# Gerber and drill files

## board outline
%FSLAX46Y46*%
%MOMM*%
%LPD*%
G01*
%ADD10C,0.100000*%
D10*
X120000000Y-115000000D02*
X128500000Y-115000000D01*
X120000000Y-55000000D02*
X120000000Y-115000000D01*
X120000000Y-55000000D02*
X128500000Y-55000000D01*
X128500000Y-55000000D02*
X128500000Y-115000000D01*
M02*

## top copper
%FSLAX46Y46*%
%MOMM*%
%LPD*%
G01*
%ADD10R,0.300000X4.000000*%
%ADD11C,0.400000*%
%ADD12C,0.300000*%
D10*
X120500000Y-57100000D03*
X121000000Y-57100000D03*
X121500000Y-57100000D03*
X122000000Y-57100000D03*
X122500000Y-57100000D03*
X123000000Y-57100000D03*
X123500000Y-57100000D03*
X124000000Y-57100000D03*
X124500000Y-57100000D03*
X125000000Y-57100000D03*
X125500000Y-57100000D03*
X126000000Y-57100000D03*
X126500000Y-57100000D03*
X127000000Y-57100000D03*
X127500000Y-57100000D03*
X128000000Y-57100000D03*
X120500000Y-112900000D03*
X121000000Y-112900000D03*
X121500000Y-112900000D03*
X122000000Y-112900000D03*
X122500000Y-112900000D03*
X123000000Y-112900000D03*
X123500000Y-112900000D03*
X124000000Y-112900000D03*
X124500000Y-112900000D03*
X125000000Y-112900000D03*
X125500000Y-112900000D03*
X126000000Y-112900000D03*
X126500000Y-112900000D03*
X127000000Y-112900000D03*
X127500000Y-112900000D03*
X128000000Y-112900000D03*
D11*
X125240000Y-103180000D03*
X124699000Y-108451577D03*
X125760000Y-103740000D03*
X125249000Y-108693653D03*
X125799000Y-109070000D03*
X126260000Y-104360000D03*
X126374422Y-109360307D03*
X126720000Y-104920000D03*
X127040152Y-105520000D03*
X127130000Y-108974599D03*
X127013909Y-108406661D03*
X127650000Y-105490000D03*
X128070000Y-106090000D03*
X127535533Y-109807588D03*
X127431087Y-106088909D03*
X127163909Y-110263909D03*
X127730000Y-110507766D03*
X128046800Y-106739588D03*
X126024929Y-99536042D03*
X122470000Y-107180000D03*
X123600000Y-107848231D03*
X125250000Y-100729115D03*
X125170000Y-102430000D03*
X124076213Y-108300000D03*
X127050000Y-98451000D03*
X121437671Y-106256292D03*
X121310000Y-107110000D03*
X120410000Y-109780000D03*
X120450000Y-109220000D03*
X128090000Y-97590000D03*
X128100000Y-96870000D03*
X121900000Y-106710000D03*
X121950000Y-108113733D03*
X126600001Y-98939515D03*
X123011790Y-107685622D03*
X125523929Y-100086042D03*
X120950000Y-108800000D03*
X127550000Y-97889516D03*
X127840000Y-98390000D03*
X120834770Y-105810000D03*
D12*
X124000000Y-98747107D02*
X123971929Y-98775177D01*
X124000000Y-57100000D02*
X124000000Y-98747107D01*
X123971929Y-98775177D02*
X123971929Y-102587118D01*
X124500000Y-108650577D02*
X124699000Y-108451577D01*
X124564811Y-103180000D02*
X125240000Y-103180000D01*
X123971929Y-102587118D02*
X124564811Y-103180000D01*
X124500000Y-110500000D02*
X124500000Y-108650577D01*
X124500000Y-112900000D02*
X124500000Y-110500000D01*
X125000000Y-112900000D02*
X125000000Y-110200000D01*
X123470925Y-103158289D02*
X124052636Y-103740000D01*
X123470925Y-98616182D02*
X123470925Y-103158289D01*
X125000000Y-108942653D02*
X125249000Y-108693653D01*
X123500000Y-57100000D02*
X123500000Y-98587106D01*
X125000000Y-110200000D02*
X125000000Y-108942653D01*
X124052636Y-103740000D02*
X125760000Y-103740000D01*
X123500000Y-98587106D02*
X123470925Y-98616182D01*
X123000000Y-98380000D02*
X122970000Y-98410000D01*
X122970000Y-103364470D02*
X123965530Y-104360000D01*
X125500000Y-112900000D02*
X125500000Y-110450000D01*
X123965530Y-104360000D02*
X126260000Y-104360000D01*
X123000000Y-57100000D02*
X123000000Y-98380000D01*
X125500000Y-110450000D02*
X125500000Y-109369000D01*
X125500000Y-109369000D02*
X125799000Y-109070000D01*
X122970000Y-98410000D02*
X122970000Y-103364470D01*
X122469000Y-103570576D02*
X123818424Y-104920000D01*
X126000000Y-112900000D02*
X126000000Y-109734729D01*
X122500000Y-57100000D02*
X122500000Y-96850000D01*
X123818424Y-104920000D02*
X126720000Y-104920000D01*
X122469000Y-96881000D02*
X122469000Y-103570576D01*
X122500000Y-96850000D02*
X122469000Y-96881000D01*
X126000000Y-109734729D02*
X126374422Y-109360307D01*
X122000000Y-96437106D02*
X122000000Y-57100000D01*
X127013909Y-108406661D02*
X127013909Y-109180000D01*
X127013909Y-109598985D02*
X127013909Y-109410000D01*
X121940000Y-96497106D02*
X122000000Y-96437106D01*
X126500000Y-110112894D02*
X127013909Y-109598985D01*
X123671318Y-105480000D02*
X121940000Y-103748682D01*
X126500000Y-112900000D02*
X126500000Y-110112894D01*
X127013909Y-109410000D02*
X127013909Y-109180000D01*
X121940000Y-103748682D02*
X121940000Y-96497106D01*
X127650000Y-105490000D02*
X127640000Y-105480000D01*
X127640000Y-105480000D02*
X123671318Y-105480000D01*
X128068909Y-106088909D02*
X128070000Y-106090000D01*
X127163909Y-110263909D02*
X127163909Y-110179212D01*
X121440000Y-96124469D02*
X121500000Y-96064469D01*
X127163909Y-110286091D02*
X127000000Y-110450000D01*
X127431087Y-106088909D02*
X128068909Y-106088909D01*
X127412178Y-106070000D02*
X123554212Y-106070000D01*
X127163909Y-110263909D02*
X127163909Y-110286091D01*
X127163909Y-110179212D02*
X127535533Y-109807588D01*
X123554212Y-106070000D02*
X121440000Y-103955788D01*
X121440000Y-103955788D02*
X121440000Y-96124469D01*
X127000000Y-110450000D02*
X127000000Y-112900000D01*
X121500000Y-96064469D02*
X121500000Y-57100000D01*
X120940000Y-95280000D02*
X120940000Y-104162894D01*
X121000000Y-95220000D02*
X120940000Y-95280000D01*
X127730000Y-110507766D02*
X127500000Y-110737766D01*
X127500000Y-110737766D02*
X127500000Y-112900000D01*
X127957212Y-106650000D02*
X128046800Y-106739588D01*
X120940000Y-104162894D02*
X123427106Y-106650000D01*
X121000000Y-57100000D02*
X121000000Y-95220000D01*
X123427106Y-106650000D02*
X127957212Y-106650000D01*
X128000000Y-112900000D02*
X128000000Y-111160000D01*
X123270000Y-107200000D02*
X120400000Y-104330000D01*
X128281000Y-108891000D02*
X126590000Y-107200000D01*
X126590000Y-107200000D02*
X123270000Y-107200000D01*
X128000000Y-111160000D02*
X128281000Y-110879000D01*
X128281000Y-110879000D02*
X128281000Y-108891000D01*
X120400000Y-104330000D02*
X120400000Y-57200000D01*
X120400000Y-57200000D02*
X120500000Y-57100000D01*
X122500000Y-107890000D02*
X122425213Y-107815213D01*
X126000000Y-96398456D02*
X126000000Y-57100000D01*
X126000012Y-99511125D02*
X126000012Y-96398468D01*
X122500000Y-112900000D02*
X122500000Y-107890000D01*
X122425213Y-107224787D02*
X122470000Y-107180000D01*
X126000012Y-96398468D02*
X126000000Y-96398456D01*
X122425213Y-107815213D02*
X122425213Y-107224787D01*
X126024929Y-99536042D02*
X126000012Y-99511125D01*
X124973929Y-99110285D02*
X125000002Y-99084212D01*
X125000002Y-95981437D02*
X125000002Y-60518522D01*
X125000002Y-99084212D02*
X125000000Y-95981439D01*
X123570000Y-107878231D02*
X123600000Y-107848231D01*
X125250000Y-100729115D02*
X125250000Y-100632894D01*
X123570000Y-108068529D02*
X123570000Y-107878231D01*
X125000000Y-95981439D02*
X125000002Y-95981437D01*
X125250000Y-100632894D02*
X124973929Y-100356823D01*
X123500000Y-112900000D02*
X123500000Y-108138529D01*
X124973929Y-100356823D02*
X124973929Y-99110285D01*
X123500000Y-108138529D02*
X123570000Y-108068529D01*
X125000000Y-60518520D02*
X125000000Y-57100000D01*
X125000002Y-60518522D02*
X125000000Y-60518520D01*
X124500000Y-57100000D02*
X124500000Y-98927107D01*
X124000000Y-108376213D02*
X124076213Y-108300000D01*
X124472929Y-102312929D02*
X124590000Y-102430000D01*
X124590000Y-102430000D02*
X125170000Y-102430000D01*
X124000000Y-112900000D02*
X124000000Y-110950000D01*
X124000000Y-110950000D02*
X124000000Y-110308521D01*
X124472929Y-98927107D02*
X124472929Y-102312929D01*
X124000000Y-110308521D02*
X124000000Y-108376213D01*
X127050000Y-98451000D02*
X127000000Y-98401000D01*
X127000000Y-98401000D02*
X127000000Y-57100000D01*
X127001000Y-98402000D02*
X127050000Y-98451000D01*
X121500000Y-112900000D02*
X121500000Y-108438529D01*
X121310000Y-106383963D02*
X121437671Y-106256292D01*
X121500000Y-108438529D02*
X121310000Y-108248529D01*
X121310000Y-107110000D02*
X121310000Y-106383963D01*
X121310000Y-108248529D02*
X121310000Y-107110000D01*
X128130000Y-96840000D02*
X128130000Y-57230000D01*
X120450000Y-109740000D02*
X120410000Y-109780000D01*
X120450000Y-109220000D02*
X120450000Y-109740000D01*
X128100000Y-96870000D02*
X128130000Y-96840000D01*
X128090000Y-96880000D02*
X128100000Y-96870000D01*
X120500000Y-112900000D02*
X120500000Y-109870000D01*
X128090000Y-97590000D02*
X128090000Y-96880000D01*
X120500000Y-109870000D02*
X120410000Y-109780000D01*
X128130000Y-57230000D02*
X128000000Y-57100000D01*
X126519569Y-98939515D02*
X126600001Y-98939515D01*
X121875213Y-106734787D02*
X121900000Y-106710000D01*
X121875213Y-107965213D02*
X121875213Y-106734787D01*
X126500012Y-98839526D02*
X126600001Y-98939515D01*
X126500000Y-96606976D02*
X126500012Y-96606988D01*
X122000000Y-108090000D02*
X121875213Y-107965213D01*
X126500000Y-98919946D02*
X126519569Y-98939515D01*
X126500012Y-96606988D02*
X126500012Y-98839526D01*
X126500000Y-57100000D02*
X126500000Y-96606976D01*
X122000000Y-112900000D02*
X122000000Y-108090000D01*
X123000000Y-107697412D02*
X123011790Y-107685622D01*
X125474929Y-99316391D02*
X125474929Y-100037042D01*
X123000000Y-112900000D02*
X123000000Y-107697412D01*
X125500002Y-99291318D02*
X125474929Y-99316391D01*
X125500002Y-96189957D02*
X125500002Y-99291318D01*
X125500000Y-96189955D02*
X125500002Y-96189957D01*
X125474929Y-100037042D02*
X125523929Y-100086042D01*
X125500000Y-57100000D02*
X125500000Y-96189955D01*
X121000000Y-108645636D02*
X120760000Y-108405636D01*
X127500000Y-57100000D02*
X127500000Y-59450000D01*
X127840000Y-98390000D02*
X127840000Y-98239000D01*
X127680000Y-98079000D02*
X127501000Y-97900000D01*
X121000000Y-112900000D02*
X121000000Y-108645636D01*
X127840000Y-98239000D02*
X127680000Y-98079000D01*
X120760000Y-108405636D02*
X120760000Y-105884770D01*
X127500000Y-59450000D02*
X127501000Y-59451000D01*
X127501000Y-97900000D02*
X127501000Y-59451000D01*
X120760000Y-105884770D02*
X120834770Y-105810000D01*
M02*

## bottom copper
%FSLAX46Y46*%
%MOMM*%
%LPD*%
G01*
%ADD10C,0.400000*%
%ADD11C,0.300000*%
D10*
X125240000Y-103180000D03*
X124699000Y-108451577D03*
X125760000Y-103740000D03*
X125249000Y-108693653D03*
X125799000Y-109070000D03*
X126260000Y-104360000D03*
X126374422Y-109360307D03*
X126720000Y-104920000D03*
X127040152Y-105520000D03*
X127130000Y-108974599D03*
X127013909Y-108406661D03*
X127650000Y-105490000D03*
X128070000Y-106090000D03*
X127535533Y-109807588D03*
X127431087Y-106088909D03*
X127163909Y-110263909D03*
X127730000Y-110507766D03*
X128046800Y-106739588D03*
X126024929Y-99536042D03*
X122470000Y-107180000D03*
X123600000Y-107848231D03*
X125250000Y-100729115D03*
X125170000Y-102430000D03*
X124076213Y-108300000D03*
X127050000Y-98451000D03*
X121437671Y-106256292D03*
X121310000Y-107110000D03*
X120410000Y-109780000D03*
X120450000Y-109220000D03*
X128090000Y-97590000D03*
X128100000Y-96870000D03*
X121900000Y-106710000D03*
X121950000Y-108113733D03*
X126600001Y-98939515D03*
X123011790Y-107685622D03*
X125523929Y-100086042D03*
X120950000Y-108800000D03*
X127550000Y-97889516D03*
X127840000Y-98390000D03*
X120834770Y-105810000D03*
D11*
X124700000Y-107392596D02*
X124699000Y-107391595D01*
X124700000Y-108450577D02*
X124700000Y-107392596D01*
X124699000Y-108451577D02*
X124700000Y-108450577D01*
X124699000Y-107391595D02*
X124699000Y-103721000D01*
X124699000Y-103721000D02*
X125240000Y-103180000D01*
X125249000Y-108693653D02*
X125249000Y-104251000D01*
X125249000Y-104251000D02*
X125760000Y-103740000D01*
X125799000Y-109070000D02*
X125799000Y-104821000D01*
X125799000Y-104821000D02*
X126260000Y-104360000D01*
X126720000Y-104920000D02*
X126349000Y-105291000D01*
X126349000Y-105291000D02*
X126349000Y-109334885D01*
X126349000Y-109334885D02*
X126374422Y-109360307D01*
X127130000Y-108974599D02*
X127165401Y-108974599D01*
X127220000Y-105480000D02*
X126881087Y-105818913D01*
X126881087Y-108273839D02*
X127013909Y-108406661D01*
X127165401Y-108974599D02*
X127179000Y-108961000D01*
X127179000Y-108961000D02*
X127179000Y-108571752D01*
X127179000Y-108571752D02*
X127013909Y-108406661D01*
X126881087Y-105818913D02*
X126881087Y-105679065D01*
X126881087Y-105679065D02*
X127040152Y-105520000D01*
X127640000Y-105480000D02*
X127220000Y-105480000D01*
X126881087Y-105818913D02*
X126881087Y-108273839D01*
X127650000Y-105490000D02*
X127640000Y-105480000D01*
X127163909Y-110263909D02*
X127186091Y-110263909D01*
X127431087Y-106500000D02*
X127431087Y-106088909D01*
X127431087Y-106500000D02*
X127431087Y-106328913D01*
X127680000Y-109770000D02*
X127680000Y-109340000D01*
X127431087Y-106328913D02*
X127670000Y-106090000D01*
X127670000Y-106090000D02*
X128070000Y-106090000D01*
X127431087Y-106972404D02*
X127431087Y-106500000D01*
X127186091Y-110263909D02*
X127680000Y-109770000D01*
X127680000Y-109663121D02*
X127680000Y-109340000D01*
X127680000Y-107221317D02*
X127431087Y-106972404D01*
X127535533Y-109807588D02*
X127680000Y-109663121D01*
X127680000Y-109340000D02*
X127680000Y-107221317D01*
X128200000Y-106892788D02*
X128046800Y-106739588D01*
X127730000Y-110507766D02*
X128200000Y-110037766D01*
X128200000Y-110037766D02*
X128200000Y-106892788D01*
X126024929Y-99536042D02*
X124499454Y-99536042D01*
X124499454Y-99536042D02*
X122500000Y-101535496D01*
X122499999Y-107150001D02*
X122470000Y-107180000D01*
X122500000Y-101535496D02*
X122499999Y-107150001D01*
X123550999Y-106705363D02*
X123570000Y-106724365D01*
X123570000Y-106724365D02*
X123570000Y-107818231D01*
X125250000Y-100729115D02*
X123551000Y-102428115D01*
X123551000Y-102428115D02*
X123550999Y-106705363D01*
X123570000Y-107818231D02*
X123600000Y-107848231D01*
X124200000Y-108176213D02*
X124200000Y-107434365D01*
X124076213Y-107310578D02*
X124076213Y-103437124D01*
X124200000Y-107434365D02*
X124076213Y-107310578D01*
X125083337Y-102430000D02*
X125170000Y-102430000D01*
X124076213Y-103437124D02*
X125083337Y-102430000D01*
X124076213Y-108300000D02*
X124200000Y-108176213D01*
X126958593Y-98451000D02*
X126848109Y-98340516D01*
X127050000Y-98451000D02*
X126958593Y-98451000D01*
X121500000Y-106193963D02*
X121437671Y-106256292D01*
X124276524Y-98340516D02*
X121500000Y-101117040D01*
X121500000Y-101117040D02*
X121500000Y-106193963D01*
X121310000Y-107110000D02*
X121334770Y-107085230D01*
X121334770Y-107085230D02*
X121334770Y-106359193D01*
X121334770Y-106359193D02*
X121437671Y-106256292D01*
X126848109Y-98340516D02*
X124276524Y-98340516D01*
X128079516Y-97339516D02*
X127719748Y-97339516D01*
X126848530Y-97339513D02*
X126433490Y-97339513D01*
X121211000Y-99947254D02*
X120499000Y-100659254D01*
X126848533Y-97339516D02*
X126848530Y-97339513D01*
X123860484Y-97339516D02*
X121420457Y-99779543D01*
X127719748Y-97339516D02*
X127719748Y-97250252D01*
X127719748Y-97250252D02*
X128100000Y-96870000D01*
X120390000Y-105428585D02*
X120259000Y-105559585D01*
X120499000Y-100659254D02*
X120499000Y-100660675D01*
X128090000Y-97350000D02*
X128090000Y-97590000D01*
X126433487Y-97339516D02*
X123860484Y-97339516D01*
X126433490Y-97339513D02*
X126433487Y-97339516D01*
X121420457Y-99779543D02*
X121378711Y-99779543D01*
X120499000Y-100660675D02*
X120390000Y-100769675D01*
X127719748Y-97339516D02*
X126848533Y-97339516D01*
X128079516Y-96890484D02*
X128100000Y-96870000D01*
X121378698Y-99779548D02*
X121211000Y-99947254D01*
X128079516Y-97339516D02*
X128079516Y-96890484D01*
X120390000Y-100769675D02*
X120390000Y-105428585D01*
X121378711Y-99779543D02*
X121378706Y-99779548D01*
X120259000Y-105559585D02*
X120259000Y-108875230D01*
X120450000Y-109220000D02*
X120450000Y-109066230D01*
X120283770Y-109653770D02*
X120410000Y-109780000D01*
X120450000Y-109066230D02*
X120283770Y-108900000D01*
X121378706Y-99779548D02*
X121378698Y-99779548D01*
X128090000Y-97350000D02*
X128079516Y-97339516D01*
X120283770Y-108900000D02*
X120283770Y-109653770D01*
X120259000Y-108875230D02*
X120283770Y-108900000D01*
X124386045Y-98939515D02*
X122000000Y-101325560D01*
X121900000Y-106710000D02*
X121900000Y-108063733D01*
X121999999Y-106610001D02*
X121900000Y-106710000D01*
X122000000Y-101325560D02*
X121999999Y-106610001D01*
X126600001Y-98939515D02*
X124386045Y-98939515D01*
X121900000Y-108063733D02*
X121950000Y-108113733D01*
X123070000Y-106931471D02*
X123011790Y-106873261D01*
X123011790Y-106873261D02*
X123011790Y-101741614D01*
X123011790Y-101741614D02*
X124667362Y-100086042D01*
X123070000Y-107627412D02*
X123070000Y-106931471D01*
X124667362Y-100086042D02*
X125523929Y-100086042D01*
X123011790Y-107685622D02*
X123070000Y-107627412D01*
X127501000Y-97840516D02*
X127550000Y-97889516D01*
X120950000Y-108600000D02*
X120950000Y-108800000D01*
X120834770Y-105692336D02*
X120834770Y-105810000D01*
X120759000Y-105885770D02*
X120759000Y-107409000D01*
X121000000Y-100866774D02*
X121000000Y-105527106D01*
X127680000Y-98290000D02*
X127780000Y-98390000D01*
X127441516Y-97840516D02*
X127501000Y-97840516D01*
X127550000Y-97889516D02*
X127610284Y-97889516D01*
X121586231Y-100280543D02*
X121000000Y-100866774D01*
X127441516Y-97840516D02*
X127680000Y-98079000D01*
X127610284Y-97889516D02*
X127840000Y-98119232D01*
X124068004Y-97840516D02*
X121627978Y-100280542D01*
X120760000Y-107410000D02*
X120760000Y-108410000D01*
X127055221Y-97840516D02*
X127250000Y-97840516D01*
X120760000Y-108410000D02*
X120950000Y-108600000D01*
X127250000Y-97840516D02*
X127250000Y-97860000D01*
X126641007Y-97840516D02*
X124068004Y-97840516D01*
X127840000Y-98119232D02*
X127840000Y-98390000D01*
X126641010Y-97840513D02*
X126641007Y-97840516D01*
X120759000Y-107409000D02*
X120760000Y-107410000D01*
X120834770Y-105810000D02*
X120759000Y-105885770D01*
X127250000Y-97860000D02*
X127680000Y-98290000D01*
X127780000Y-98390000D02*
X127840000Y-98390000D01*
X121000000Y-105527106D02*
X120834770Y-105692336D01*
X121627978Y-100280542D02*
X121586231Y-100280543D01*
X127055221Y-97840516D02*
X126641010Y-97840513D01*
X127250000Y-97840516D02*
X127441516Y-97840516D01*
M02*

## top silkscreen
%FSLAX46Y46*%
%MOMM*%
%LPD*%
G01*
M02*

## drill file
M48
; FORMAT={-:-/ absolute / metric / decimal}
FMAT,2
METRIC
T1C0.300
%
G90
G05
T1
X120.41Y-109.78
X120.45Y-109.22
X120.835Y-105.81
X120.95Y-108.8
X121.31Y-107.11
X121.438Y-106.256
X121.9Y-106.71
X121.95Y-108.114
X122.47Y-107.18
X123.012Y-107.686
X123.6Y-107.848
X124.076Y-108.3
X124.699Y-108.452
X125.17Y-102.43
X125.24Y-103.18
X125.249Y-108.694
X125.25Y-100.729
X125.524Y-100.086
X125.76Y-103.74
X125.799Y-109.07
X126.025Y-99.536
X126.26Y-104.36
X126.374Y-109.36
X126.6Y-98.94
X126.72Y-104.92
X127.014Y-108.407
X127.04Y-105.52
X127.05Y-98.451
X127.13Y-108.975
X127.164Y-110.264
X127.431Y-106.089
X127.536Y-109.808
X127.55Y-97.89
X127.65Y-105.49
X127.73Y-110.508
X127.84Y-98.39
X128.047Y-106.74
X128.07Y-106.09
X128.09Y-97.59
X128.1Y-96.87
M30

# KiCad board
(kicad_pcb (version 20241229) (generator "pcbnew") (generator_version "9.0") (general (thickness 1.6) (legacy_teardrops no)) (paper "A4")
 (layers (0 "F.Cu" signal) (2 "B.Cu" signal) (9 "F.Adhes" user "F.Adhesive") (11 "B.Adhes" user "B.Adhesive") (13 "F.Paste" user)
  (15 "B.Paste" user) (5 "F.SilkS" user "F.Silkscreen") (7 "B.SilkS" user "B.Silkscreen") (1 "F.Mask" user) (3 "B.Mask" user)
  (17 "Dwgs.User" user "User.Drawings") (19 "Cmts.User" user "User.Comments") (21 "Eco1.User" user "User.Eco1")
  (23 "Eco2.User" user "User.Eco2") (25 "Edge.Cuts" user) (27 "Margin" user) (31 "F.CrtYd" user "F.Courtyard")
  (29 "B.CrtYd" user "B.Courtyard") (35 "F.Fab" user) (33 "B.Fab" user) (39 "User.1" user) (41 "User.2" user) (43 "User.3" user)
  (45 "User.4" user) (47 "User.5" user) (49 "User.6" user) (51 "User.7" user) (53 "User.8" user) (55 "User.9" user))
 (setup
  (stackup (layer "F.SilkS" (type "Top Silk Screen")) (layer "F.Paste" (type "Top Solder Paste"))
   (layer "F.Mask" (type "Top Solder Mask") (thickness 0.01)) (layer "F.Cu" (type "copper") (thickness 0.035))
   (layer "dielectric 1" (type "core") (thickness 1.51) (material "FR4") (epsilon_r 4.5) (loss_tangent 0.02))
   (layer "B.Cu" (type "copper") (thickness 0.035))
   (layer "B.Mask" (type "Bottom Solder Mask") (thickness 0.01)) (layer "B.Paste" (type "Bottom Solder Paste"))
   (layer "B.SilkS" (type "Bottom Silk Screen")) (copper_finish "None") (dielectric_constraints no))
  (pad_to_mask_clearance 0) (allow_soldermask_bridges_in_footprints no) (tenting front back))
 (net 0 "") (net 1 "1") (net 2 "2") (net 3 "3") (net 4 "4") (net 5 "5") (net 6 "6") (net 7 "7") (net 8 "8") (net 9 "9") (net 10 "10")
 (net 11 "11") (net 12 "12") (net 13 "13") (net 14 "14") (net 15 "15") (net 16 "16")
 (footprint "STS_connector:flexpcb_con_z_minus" (layer "F.Cu") (at 120 59.1)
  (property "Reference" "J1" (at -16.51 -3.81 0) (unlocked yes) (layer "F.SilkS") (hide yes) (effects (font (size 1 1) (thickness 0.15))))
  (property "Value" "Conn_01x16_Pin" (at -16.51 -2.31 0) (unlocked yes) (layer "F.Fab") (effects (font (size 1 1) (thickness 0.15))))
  (pad "1" smd rect (at 0.5 -2) (size 0.3 4) (layers "F.Cu" "F.Mask" "F.Paste") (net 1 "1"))
  (pad "2" smd rect (at 1 -2) (size 0.3 4) (layers "F.Cu" "F.Mask" "F.Paste") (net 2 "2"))
  (pad "3" smd rect (at 1.5 -2) (size 0.3 4) (layers "F.Cu" "F.Mask" "F.Paste") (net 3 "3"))
  (pad "4" smd rect (at 2 -2) (size 0.3 4) (layers "F.Cu" "F.Mask" "F.Paste") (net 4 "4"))
  (pad "5" smd rect (at 2.5 -2) (size 0.3 4) (layers "F.Cu" "F.Mask" "F.Paste") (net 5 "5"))
  (pad "6" smd rect (at 3 -2) (size 0.3 4) (layers "F.Cu" "F.Mask" "F.Paste") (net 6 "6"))
  (pad "7" smd rect (at 3.5 -2) (size 0.3 4) (layers "F.Cu" "F.Mask" "F.Paste") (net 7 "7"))
  (pad "8" smd rect (at 4 -2) (size 0.3 4) (layers "F.Cu" "F.Mask" "F.Paste") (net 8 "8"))
  (pad "9" smd rect (at 4.5 -2) (size 0.3 4) (layers "F.Cu" "F.Mask" "F.Paste") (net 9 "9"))
  (pad "10" smd rect (at 5 -2) (size 0.3 4) (layers "F.Cu" "F.Mask" "F.Paste") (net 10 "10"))
  (pad "11" smd rect (at 5.5 -2) (size 0.3 4) (layers "F.Cu" "F.Mask" "F.Paste") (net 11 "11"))
  (pad "12" smd rect (at 6 -2) (size 0.3 4) (layers "F.Cu" "F.Mask" "F.Paste") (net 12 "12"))
  (pad "13" smd rect (at 6.5 -2) (size 0.3 4) (layers "F.Cu" "F.Mask" "F.Paste") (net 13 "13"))
  (pad "14" smd rect (at 7 -2) (size 0.3 4) (layers "F.Cu" "F.Mask" "F.Paste") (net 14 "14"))
  (pad "15" smd rect (at 7.5 -2) (size 0.3 4) (layers "F.Cu" "F.Mask" "F.Paste") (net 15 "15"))
  (pad "16" smd rect (at 8 -2) (size 0.3 4) (layers "F.Cu" "F.Mask" "F.Paste") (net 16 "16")))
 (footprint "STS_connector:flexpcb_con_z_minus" (layer "F.Cu") (at 120 114.9)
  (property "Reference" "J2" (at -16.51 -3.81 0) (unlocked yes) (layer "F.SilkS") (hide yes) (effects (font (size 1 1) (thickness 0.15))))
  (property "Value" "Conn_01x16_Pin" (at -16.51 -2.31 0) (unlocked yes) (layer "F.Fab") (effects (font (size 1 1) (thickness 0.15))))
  (pad "1" smd rect (at 0.5 -2) (size 0.3 4) (layers "F.Cu" "F.Mask" "F.Paste") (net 16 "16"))
  (pad "2" smd rect (at 1 -2) (size 0.3 4) (layers "F.Cu" "F.Mask" "F.Paste") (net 15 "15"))
  (pad "3" smd rect (at 1.5 -2) (size 0.3 4) (layers "F.Cu" "F.Mask" "F.Paste") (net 14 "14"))
  (pad "4" smd rect (at 2 -2) (size 0.3 4) (layers "F.Cu" "F.Mask" "F.Paste") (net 13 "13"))
  (pad "5" smd rect (at 2.5 -2) (size 0.3 4) (layers "F.Cu" "F.Mask" "F.Paste") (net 12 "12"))
  (pad "6" smd rect (at 3 -2) (size 0.3 4) (layers "F.Cu" "F.Mask" "F.Paste") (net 11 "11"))
  (pad "7" smd rect (at 3.5 -2) (size 0.3 4) (layers "F.Cu" "F.Mask" "F.Paste") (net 10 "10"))
  (pad "8" smd rect (at 4 -2) (size 0.3 4) (layers "F.Cu" "F.Mask" "F.Paste") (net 9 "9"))
  (pad "9" smd rect (at 4.5 -2) (size 0.3 4) (layers "F.Cu" "F.Mask" "F.Paste") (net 8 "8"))
  (pad "10" smd rect (at 5 -2) (size 0.3 4) (layers "F.Cu" "F.Mask" "F.Paste") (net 7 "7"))
  (pad "11" smd rect (at 5.5 -2) (size 0.3 4) (layers "F.Cu" "F.Mask" "F.Paste") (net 6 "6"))
  (pad "12" smd rect (at 6 -2) (size 0.3 4) (layers "F.Cu" "F.Mask" "F.Paste") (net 5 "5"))
  (pad "13" smd rect (at 6.5 -2) (size 0.3 4) (layers "F.Cu" "F.Mask" "F.Paste") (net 4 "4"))
  (pad "14" smd rect (at 7 -2) (size 0.3 4) (layers "F.Cu" "F.Mask" "F.Paste") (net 3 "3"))
  (pad "15" smd rect (at 7.5 -2) (size 0.3 4) (layers "F.Cu" "F.Mask" "F.Paste") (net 2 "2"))
  (pad "16" smd rect (at 8 -2) (size 0.3 4) (layers "F.Cu" "F.Mask" "F.Paste") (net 1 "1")))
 (gr_line (start 120 115) (end 128.5 115) (stroke (width 0.1) (type solid)) (layer "Edge.Cuts"))
 (gr_line (start 120 55) (end 120 115) (stroke (width 0.1) (type solid)) (layer "Edge.Cuts"))
 (gr_line (start 120 55) (end 128.5 55) (stroke (width 0.1) (type solid)) (layer "Edge.Cuts"))
 (gr_line (start 128.5 55) (end 128.5 115) (stroke (width 0.1) (type solid)) (layer "Edge.Cuts"))
 (segment (start 124 98.747107) (end 123.971929 98.775177) (width 0.3) (layer "F.Cu") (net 8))
 (segment (start 124 57.1) (end 124 98.747107) (width 0.3) (layer "F.Cu") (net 8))
 (segment (start 123.971929 98.775177) (end 123.971929 102.587118) (width 0.3) (layer "F.Cu") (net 8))
 (segment (start 124.5 108.650577) (end 124.699 108.451577) (width 0.3) (layer "F.Cu") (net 8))
 (segment (start 124.564811 103.18) (end 125.24 103.18) (width 0.3) (layer "F.Cu") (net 8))
 (segment (start 123.971929 102.587118) (end 124.564811 103.18) (width 0.3) (layer "F.Cu") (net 8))
 (segment (start 124.5 110.5) (end 124.5 108.650577) (width 0.3) (layer "F.Cu") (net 8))
 (segment (start 124.5 112.9) (end 124.5 110.5) (width 0.3) (layer "F.Cu") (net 8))
 (via (at 125.24 103.18) (size 0.4) (drill 0.3) (layers "F.Cu" "B.Cu") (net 8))
 (via (at 124.699 108.451577) (size 0.4) (drill 0.3) (layers "F.Cu" "B.Cu") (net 8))
 (segment (start 124.7 107.392596) (end 124.699 107.391595) (width 0.3) (layer "B.Cu") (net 8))
 (segment (start 124.7 108.450577) (end 124.7 107.392596) (width 0.3) (layer "B.Cu") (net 8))
 (segment (start 124.699 108.451577) (end 124.7 108.450577) (width 0.3) (layer "B.Cu") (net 8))
 (segment (start 124.699 107.391595) (end 124.699 103.721) (width 0.3) (layer "B.Cu") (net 8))
 (segment (start 124.699 103.721) (end 125.24 103.18) (width 0.3) (layer "B.Cu") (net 8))
 (segment (start 125 112.9) (end 125 110.2) (width 0.3) (layer "F.Cu") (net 7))
 (segment (start 123.470925 103.158289) (end 124.052636 103.74) (width 0.3) (layer "F.Cu") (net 7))
 (segment (start 123.470925 98.616182) (end 123.470925 103.158289) (width 0.3) (layer "F.Cu") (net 7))
 (segment (start 125 108.942653) (end 125.249 108.693653) (width 0.3) (layer "F.Cu") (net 7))
 (segment (start 123.5 57.1) (end 123.5 98.587106) (width 0.3) (layer "F.Cu") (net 7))
 (segment (start 125 110.2) (end 125 108.942653) (width 0.3) (layer "F.Cu") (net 7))
 (segment (start 124.052636 103.74) (end 125.76 103.74) (width 0.3) (layer "F.Cu") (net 7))
 (segment (start 123.5 98.587106) (end 123.470925 98.616182) (width 0.3) (layer "F.Cu") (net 7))
 (via (at 125.76 103.74) (size 0.4) (drill 0.3) (layers "F.Cu" "B.Cu") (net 7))
 (via (at 125.249 108.693653) (size 0.4) (drill 0.3) (layers "F.Cu" "B.Cu") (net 7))
 (segment (start 125.249 108.693653) (end 125.249 104.251) (width 0.3) (layer "B.Cu") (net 7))
 (segment (start 125.249 104.251) (end 125.76 103.74) (width 0.3) (layer "B.Cu") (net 7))
 (segment (start 123 98.38) (end 122.97 98.41) (width 0.3) (layer "F.Cu") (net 6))
 (segment (start 122.97 103.36447) (end 123.96553 104.36) (width 0.3) (layer "F.Cu") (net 6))
 (segment (start 125.5 112.9) (end 125.5 110.45) (width 0.3) (layer "F.Cu") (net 6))
 (segment (start 123.96553 104.36) (end 126.26 104.36) (width 0.3) (layer "F.Cu") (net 6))
 (segment (start 123 57.1) (end 123 98.38) (width 0.3) (layer "F.Cu") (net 6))
 (segment (start 125.5 110.45) (end 125.5 109.369) (width 0.3) (layer "F.Cu") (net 6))
 (segment (start 125.5 109.369) (end 125.799 109.07) (width 0.3) (layer "F.Cu") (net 6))
 (segment (start 122.97 98.41) (end 122.97 103.36447) (width 0.3) (layer "F.Cu") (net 6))
 (via (at 125.799 109.07) (size 0.4) (drill 0.3) (layers "F.Cu" "B.Cu") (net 6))
 (via (at 126.26 104.36) (size 0.4) (drill 0.3) (layers "F.Cu" "B.Cu") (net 6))
 (segment (start 125.799 109.07) (end 125.799 104.821) (width 0.3) (layer "B.Cu") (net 6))
 (segment (start 125.799 104.821) (end 126.26 104.36) (width 0.3) (layer "B.Cu") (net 6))
 (segment (start 122.469 103.570576) (end 123.818424 104.92) (width 0.3) (layer "F.Cu") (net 5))
 (segment (start 126 112.9) (end 126 109.734729) (width 0.3) (layer "F.Cu") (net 5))
 (segment (start 122.5 57.1) (end 122.5 96.85) (width 0.3) (layer "F.Cu") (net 5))
 (segment (start 123.818424 104.92) (end 126.72 104.92) (width 0.3) (layer "F.Cu") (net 5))
 (segment (start 122.469 96.881) (end 122.469 103.570576) (width 0.3) (layer "F.Cu") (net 5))
 (segment (start 122.5 96.85) (end 122.469 96.881) (width 0.3) (layer "F.Cu") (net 5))
 (segment (start 126 109.734729) (end 126.374422 109.360307) (width 0.3) (layer "F.Cu") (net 5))
 (via (at 126.374422 109.360307) (size 0.4) (drill 0.3) (layers "F.Cu" "B.Cu") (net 5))
 (via (at 126.72 104.92) (size 0.4) (drill 0.3) (layers "F.Cu" "B.Cu") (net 5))
 (segment (start 126.72 104.92) (end 126.349 105.291) (width 0.3) (layer "B.Cu") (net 5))
 (segment (start 126.349 105.291) (end 126.349 109.334885) (width 0.3) (layer "B.Cu") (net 5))
 (segment (start 126.349 109.334885) (end 126.374422 109.360307) (width 0.3) (layer "B.Cu") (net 5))
 (segment (start 122 96.437106) (end 122 57.1) (width 0.3) (layer "F.Cu") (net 4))
 (segment (start 127.013909 108.406661) (end 127.013909 109.18) (width 0.3) (layer "F.Cu") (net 4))
 (segment (start 127.013909 109.598985) (end 127.013909 109.41) (width 0.3) (layer "F.Cu") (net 4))
 (segment (start 121.94 96.497106) (end 122 96.437106) (width 0.3) (layer "F.Cu") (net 4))
 (segment (start 126.5 110.112894) (end 127.013909 109.598985) (width 0.3) (layer "F.Cu") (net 4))
 (segment (start 123.671318 105.48) (end 121.94 103.748682) (width 0.3) (layer "F.Cu") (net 4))
 (segment (start 126.5 112.9) (end 126.5 110.112894) (width 0.3) (layer "F.Cu") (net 4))
 (segment (start 127.013909 109.41) (end 127.013909 109.18) (width 0.3) (layer "F.Cu") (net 4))
 (segment (start 121.94 103.748682) (end 121.94 96.497106) (width 0.3) (layer "F.Cu") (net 4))
 (segment (start 127.65 105.49) (end 127.64 105.48) (width 0.3) (layer "F.Cu") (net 4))
 (segment (start 127.64 105.48) (end 123.671318 105.48) (width 0.3) (layer "F.Cu") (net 4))
 (via (at 127.040152 105.52) (size 0.4) (drill 0.3) (layers "F.Cu" "B.Cu") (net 4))
 (via (at 127.13 108.974599) (size 0.4) (drill 0.3) (layers "F.Cu" "B.Cu") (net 4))
 (via (at 127.013909 108.406661) (size 0.4) (drill 0.3) (layers "F.Cu" "B.Cu") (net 4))
 (via (at 127.65 105.49) (size 0.4) (drill 0.3) (layers "F.Cu" "B.Cu") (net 4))
 (segment (start 127.13 108.974599) (end 127.165401 108.974599) (width 0.3) (layer "B.Cu") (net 4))
 (segment (start 127.22 105.48) (end 126.881087 105.818913) (width 0.3) (layer "B.Cu") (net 4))
 (segment (start 126.881087 108.273839) (end 127.013909 108.406661) (width 0.3) (layer "B.Cu") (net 4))
 (segment (start 127.165401 108.974599) (end 127.179 108.961) (width 0.3) (layer "B.Cu") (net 4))
 (segment (start 127.179 108.961) (end 127.179 108.571752) (width 0.3) (layer "B.Cu") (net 4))
 (segment (start 127.179 108.571752) (end 127.013909 108.406661) (width 0.3) (layer "B.Cu") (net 4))
 (segment (start 126.881087 105.818913) (end 126.881087 105.679065) (width 0.3) (layer "B.Cu") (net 4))
 (segment (start 126.881087 105.679065) (end 127.040152 105.52) (width 0.3) (layer "B.Cu") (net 4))
 (segment (start 127.64 105.48) (end 127.22 105.48) (width 0.3) (layer "B.Cu") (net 4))
 (segment (start 126.881087 105.818913) (end 126.881087 108.273839) (width 0.3) (layer "B.Cu") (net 4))
 (segment (start 127.65 105.49) (end 127.64 105.48) (width 0.3) (layer "B.Cu") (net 4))
 (segment (start 128.068909 106.088909) (end 128.07 106.09) (width 0.3) (layer "F.Cu") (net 3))
 (segment (start 127.163909 110.263909) (end 127.163909 110.179212) (width 0.3) (layer "F.Cu") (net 3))
 (segment (start 121.44 96.124469) (end 121.5 96.064469) (width 0.3) (layer "F.Cu") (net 3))
 (segment (start 127.163909 110.286091) (end 127 110.45) (width 0.3) (layer "F.Cu") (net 3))
 (segment (start 127.431087 106.088909) (end 128.068909 106.088909) (width 0.3) (layer "F.Cu") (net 3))
 (segment (start 127.412178 106.07) (end 123.554212 106.07) (width 0.3) (layer "F.Cu") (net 3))
 (segment (start 127.163909 110.263909) (end 127.163909 110.286091) (width 0.3) (layer "F.Cu") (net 3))
 (segment (start 127.163909 110.179212) (end 127.535533 109.807588) (width 0.3) (layer "F.Cu") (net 3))
 (segment (start 123.554212 106.07) (end 121.44 103.955788) (width 0.3) (layer "F.Cu") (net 3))
 (segment (start 121.44 103.955788) (end 121.44 96.124469) (width 0.3) (layer "F.Cu") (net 3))
 (segment (start 127 110.45) (end 127 112.9) (width 0.3) (layer "F.Cu") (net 3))
 (segment (start 121.5 96.064469) (end 121.5 57.1) (width 0.3) (layer "F.Cu") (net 3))
 (via (at 128.07 106.09) (size 0.4) (drill 0.3) (layers "F.Cu" "B.Cu") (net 3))
 (via (at 127.535533 109.807588) (size 0.4) (drill 0.3) (layers "F.Cu" "B.Cu") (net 3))
 (via (at 127.431087 106.088909) (size 0.4) (drill 0.3) (layers "F.Cu" "B.Cu") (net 3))
 (via (at 127.163909 110.263909) (size 0.4) (drill 0.3) (layers "F.Cu" "B.Cu") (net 3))
 (segment (start 127.163909 110.263909) (end 127.186091 110.263909) (width 0.3) (layer "B.Cu") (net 3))
 (segment (start 127.431087 106.5) (end 127.431087 106.088909) (width 0.3) (layer "B.Cu") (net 3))
 (segment (start 127.431087 106.5) (end 127.431087 106.328913) (width 0.3) (layer "B.Cu") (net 3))
 (segment (start 127.68 109.77) (end 127.68 109.34) (width 0.3) (layer "B.Cu") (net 3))
 (segment (start 127.431087 106.328913) (end 127.67 106.09) (width 0.3) (layer "B.Cu") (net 3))
 (segment (start 127.67 106.09) (end 128.07 106.09) (width 0.3) (layer "B.Cu") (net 3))
 (segment (start 127.431087 106.972404) (end 127.431087 106.5) (width 0.3) (layer "B.Cu") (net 3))
 (segment (start 127.186091 110.263909) (end 127.68 109.77) (width 0.3) (layer "B.Cu") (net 3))
 (segment (start 127.68 109.663121) (end 127.68 109.34) (width 0.3) (layer "B.Cu") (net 3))
 (segment (start 127.68 107.221317) (end 127.431087 106.972404) (width 0.3) (layer "B.Cu") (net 3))
 (segment (start 127.535533 109.807588) (end 127.68 109.663121) (width 0.3) (layer "B.Cu") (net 3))
 (segment (start 127.68 109.34) (end 127.68 107.221317) (width 0.3) (layer "B.Cu") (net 3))
 (segment (start 120.94 95.28) (end 120.94 104.162894) (width 0.3) (layer "F.Cu") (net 2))
 (segment (start 121 95.22) (end 120.94 95.28) (width 0.3) (layer "F.Cu") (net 2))
 (segment (start 127.73 110.507766) (end 127.5 110.737766) (width 0.3) (layer "F.Cu") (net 2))
 (segment (start 127.5 110.737766) (end 127.5 112.9) (width 0.3) (layer "F.Cu") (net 2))
 (segment (start 127.957212 106.65) (end 128.0468 106.739588) (width 0.3) (layer "F.Cu") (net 2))
 (segment (start 120.94 104.162894) (end 123.427106 106.65) (width 0.3) (layer "F.Cu") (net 2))
 (segment (start 121 57.1) (end 121 95.22) (width 0.3) (layer "F.Cu") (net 2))
 (segment (start 123.427106 106.65) (end 127.957212 106.65) (width 0.3) (layer "F.Cu") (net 2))
 (via (at 127.73 110.507766) (size 0.4) (drill 0.3) (layers "F.Cu" "B.Cu") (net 2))
 (via (at 128.0468 106.739588) (size 0.4) (drill 0.3) (layers "F.Cu" "B.Cu") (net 2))
 (segment (start 128.2 106.892788) (end 128.0468 106.739588) (width 0.3) (layer "B.Cu") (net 2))
 (segment (start 127.73 110.507766) (end 128.2 110.037766) (width 0.3) (layer "B.Cu") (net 2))
 (segment (start 128.2 110.037766) (end 128.2 106.892788) (width 0.3) (layer "B.Cu") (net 2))
 (segment (start 128 112.9) (end 128 111.16) (width 0.3) (layer "F.Cu") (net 1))
 (segment (start 123.27 107.2) (end 120.4 104.33) (width 0.3) (layer "F.Cu") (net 1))
 (segment (start 128.281 108.891) (end 126.59 107.2) (width 0.3) (layer "F.Cu") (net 1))
 (segment (start 126.59 107.2) (end 123.27 107.2) (width 0.3) (layer "F.Cu") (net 1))
 (segment (start 128 111.16) (end 128.281 110.879) (width 0.3) (layer "F.Cu") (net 1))
 (segment (start 128.281 110.879) (end 128.281 108.891) (width 0.3) (layer "F.Cu") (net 1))
 (segment (start 120.4 104.33) (end 120.4 57.2) (width 0.3) (layer "F.Cu") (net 1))
 (segment (start 120.4 57.2) (end 120.5 57.1) (width 0.3) (layer "F.Cu") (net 1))
 (segment (start 122.5 107.89) (end 122.425213 107.815213) (width 0.3) (layer "F.Cu") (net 12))
 (segment (start 126 96.398456) (end 126 57.1) (width 0.3) (layer "F.Cu") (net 12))
 (segment (start 126.000012 99.511125) (end 126.000012 96.398468) (width 0.3) (layer "F.Cu") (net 12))
 (segment (start 122.5 112.9) (end 122.5 107.89) (width 0.3) (layer "F.Cu") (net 12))
 (segment (start 122.425213 107.224787) (end 122.47 107.18) (width 0.3) (layer "F.Cu") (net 12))
 (segment (start 126.000012 96.398468) (end 126 96.398456) (width 0.3) (layer "F.Cu") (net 12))
 (segment (start 122.425213 107.815213) (end 122.425213 107.224787) (width 0.3) (layer "F.Cu") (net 12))
 (segment (start 126.024929 99.536042) (end 126.000012 99.511125) (width 0.3) (layer "F.Cu") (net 12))
 (via (at 126.024929 99.536042) (size 0.4) (drill 0.3) (layers "F.Cu" "B.Cu") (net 12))
 (via (at 122.47 107.18) (size 0.4) (drill 0.3) (layers "F.Cu" "B.Cu") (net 12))
 (segment (start 126.024929 99.536042) (end 124.499454 99.536042) (width 0.3) (layer "B.Cu") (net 12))
 (segment (start 124.499454 99.536042) (end 122.5 101.535496) (width 0.3) (layer "B.Cu") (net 12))
 (segment (start 122.499999 107.150001) (end 122.47 107.18) (width 0.3) (layer "B.Cu") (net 12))
 (segment (start 122.5 101.535496) (end 122.499999 107.150001) (width 0.3) (layer "B.Cu") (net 12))
 (segment (start 124.973929 99.110285) (end 125.000002 99.084212) (width 0.3) (layer "F.Cu") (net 10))
 (segment (start 125.000002 95.981437) (end 125.000002 60.518522) (width 0.3) (layer "F.Cu") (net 10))
 (segment (start 125.000002 99.084212) (end 125 95.981439) (width 0.3) (layer "F.Cu") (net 10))
 (segment (start 123.57 107.878231) (end 123.6 107.848231) (width 0.3) (layer "F.Cu") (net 10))
 (segment (start 125.25 100.729115) (end 125.25 100.632894) (width 0.3) (layer "F.Cu") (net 10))
 (segment (start 123.57 108.068529) (end 123.57 107.878231) (width 0.3) (layer "F.Cu") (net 10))
 (segment (start 125 95.981439) (end 125.000002 95.981437) (width 0.3) (layer "F.Cu") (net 10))
 (segment (start 125.25 100.632894) (end 124.973929 100.356823) (width 0.3) (layer "F.Cu") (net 10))
 (segment (start 123.5 112.9) (end 123.5 108.138529) (width 0.3) (layer "F.Cu") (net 10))
 (segment (start 124.973929 100.356823) (end 124.973929 99.110285) (width 0.3) (layer "F.Cu") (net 10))
 (segment (start 123.5 108.138529) (end 123.57 108.068529) (width 0.3) (layer "F.Cu") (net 10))
 (segment (start 125 60.51852) (end 125 57.1) (width 0.3) (layer "F.Cu") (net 10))
 (segment (start 125.000002 60.518522) (end 125 60.51852) (width 0.3) (layer "F.Cu") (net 10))
 (via (at 123.6 107.848231) (size 0.4) (drill 0.3) (layers "F.Cu" "B.Cu") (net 10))
 (via (at 125.25 100.729115) (size 0.4) (drill 0.3) (layers "F.Cu" "B.Cu") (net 10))
 (segment (start 123.550999 106.705363) (end 123.57 106.724365) (width 0.3) (layer "B.Cu") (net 10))
 (segment (start 123.57 106.724365) (end 123.57 107.818231) (width 0.3) (layer "B.Cu") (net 10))
 (segment (start 125.25 100.729115) (end 123.551 102.428115) (width 0.3) (layer "B.Cu") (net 10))
 (segment (start 123.551 102.428115) (end 123.550999 106.705363) (width 0.3) (layer "B.Cu") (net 10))
 (segment (start 123.57 107.818231) (end 123.6 107.848231) (width 0.3) (layer "B.Cu") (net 10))
 (segment (start 124.5 57.1) (end 124.5 98.927107) (width 0.3) (layer "F.Cu") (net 9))
 (segment (start 124 108.376213) (end 124.076213 108.3) (width 0.3) (layer "F.Cu") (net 9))
 (segment (start 124.472929 102.312929) (end 124.59 102.43) (width 0.3) (layer "F.Cu") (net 9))
 (segment (start 124.59 102.43) (end 125.17 102.43) (width 0.3) (layer "F.Cu") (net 9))
 (segment (start 124 112.9) (end 124 110.95) (width 0.3) (layer "F.Cu") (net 9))
 (segment (start 124 110.95) (end 124 110.308521) (width 0.3) (layer "F.Cu") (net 9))
 (segment (start 124.472929 98.927107) (end 124.472929 102.312929) (width 0.3) (layer "F.Cu") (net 9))
 (segment (start 124 110.308521) (end 124 108.376213) (width 0.3) (layer "F.Cu") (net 9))
 (via (at 125.17 102.43) (size 0.4) (drill 0.3) (layers "F.Cu" "B.Cu") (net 9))
 (via (at 124.076213 108.3) (size 0.4) (drill 0.3) (layers "F.Cu" "B.Cu") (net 9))
 (segment (start 124.2 108.176213) (end 124.2 107.434365) (width 0.3) (layer "B.Cu") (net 9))
 (segment (start 124.076213 107.310578) (end 124.076213 103.437124) (width 0.3) (layer "B.Cu") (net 9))
 (segment (start 124.2 107.434365) (end 124.076213 107.310578) (width 0.3) (layer "B.Cu") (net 9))
 (segment (start 125.083337 102.43) (end 125.17 102.43) (width 0.3) (layer "B.Cu") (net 9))
 (segment (start 124.076213 103.437124) (end 125.083337 102.43) (width 0.3) (layer "B.Cu") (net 9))
 (segment (start 124.076213 108.3) (end 124.2 108.176213) (width 0.3) (layer "B.Cu") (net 9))
 (segment (start 127.05 98.451) (end 127 98.401) (width 0.3) (layer "F.Cu") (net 14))
 (segment (start 127 98.401) (end 127 57.1) (width 0.3) (layer "F.Cu") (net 14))
 (segment (start 127.001 98.402) (end 127.05 98.451) (width 0.3) (layer "F.Cu") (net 14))
 (segment (start 121.5 112.9) (end 121.5 108.438529) (width 0.3) (layer "F.Cu") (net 14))
 (segment (start 121.31 106.383963) (end 121.437671 106.256292) (width 0.3) (layer "F.Cu") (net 14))
 (segment (start 121.5 108.438529) (end 121.31 108.248529) (width 0.3) (layer "F.Cu") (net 14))
 (segment (start 121.31 107.11) (end 121.31 106.383963) (width 0.3) (layer "F.Cu") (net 14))
 (segment (start 121.31 108.248529) (end 121.31 107.11) (width 0.3) (layer "F.Cu") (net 14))
 (via (at 127.05 98.451) (size 0.4) (drill 0.3) (layers "F.Cu" "B.Cu") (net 14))
 (via (at 121.437671 106.256292) (size 0.4) (drill 0.3) (layers "F.Cu" "B.Cu") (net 14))
 (via (at 121.31 107.11) (size 0.4) (drill 0.3) (layers "F.Cu" "B.Cu") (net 14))
 (segment (start 126.958593 98.451) (end 126.848109 98.340516) (width 0.3) (layer "B.Cu") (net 14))
 (segment (start 127.05 98.451) (end 126.958593 98.451) (width 0.3) (layer "B.Cu") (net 14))
 (segment (start 121.5 106.193963) (end 121.437671 106.256292) (width 0.3) (layer "B.Cu") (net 14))
 (segment (start 124.276524 98.340516) (end 121.5 101.11704) (width 0.3) (layer "B.Cu") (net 14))
 (segment (start 121.5 101.11704) (end 121.5 106.193963) (width 0.3) (layer "B.Cu") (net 14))
 (segment (start 121.31 107.11) (end 121.33477 107.08523) (width 0.3) (layer "B.Cu") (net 14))
 (segment (start 121.33477 107.08523) (end 121.33477 106.359193) (width 0.3) (layer "B.Cu") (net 14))
 (segment (start 121.33477 106.359193) (end 121.437671 106.256292) (width 0.3) (layer "B.Cu") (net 14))
 (segment (start 126.848109 98.340516) (end 124.276524 98.340516) (width 0.3) (layer "B.Cu") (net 14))
 (segment (start 128.13 96.84) (end 128.13 57.23) (width 0.3) (layer "F.Cu") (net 16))
 (segment (start 120.45 109.74) (end 120.41 109.78) (width 0.3) (layer "F.Cu") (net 16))
 (segment (start 120.45 109.22) (end 120.45 109.74) (width 0.3) (layer "F.Cu") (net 16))
 (segment (start 128.1 96.87) (end 128.13 96.84) (width 0.3) (layer "F.Cu") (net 16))
 (segment (start 128.09 96.88) (end 128.1 96.87) (width 0.3) (layer "F.Cu") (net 16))
 (segment (start 120.5 112.9) (end 120.5 109.87) (width 0.3) (layer "F.Cu") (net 16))
 (segment (start 128.09 97.59) (end 128.09 96.88) (width 0.3) (layer "F.Cu") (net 16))
 (segment (start 120.5 109.87) (end 120.41 109.78) (width 0.3) (layer "F.Cu") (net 16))
 (segment (start 128.13 57.23) (end 128 57.1) (width 0.3) (layer "F.Cu") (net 16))
 (via (at 120.41 109.78) (size 0.4) (drill 0.3) (layers "F.Cu" "B.Cu") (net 16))
 (via (at 120.45 109.22) (size 0.4) (drill 0.3) (layers "F.Cu" "B.Cu") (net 16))
 (via (at 128.09 97.59) (size 0.4) (drill 0.3) (layers "F.Cu" "B.Cu") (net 16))
 (via (at 128.1 96.87) (size 0.4) (drill 0.3) (layers "F.Cu" "B.Cu") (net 16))
 (segment (start 128.079516 97.339516) (end 127.719748 97.339516) (width 0.3) (layer "B.Cu") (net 16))
 (segment (start 126.84853 97.339513) (end 126.43349 97.339513) (width 0.3) (layer "B.Cu") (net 16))
 (segment (start 121.211 99.947254) (end 120.499 100.659254) (width 0.3) (layer "B.Cu") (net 16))
 (segment (start 126.848533 97.339516) (end 126.84853 97.339513) (width 0.3) (layer "B.Cu") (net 16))
 (segment (start 123.860484 97.339516) (end 121.420457 99.779543) (width 0.3) (layer "B.Cu") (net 16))
 (segment (start 127.719748 97.339516) (end 127.719748 97.250252) (width 0.3) (layer "B.Cu") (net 16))
 (segment (start 127.719748 97.250252) (end 128.1 96.87) (width 0.3) (layer "B.Cu") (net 16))
 (segment (start 120.39 105.428585) (end 120.259 105.559585) (width 0.3) (layer "B.Cu") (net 16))
 (segment (start 120.499 100.659254) (end 120.499 100.660675) (width 0.3) (layer "B.Cu") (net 16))
 (segment (start 128.09 97.35) (end 128.09 97.59) (width 0.3) (layer "B.Cu") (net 16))
 (segment (start 126.433487 97.339516) (end 123.860484 97.339516) (width 0.3) (layer "B.Cu") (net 16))
 (segment (start 126.43349 97.339513) (end 126.433487 97.339516) (width 0.3) (layer "B.Cu") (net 16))
 (segment (start 121.420457 99.779543) (end 121.378711 99.779543) (width 0.3) (layer "B.Cu") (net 16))
 (segment (start 120.499 100.660675) (end 120.39 100.769675) (width 0.3) (layer "B.Cu") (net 16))
 (segment (start 127.719748 97.339516) (end 126.848533 97.339516) (width 0.3) (layer "B.Cu") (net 16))
 (segment (start 128.079516 96.890484) (end 128.1 96.87) (width 0.3) (layer "B.Cu") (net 16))
 (segment (start 121.378698 99.779548) (end 121.211 99.947254) (width 0.3) (layer "B.Cu") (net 16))
 (segment (start 128.079516 97.339516) (end 128.079516 96.890484) (width 0.3) (layer "B.Cu") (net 16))
 (segment (start 120.39 100.769675) (end 120.39 105.428585) (width 0.3) (layer "B.Cu") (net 16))
 (segment (start 121.378711 99.779543) (end 121.378706 99.779548) (width 0.3) (layer "B.Cu") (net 16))
 (segment (start 120.259 105.559585) (end 120.259 108.87523) (width 0.3) (layer "B.Cu") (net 16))
 (segment (start 120.45 109.22) (end 120.45 109.06623) (width 0.3) (layer "B.Cu") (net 16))
 (segment (start 120.28377 109.65377) (end 120.41 109.78) (width 0.3) (layer "B.Cu") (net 16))
 (segment (start 120.45 109.06623) (end 120.28377 108.9) (width 0.3) (layer "B.Cu") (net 16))
 (segment (start 121.378706 99.779548) (end 121.378698 99.779548) (width 0.3) (layer "B.Cu") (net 16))
 (segment (start 128.09 97.35) (end 128.079516 97.339516) (width 0.3) (layer "B.Cu") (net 16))
 (segment (start 120.28377 108.9) (end 120.28377 109.65377) (width 0.3) (layer "B.Cu") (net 16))
 (segment (start 120.259 108.87523) (end 120.28377 108.9) (width 0.3) (layer "B.Cu") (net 16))
 (segment (start 126.519569 98.939515) (end 126.600001 98.939515) (width 0.3) (layer "F.Cu") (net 13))
 (segment (start 121.875213 106.734787) (end 121.9 106.71) (width 0.3) (layer "F.Cu") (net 13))
 (segment (start 121.875213 107.965213) (end 121.875213 106.734787) (width 0.3) (layer "F.Cu") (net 13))
 (segment (start 126.500012 98.839526) (end 126.600001 98.939515) (width 0.3) (layer "F.Cu") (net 13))
 (segment (start 126.5 96.606976) (end 126.500012 96.606988) (width 0.3) (layer "F.Cu") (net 13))
 (segment (start 122 108.09) (end 121.875213 107.965213) (width 0.3) (layer "F.Cu") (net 13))
 (segment (start 126.5 98.919946) (end 126.519569 98.939515) (width 0.3) (layer "F.Cu") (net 13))
 (segment (start 126.500012 96.606988) (end 126.500012 98.839526) (width 0.3) (layer "F.Cu") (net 13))
 (segment (start 126.5 57.1) (end 126.5 96.606976) (width 0.3) (layer "F.Cu") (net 13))
 (segment (start 122 112.9) (end 122 108.09) (width 0.3) (layer "F.Cu") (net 13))
 (via (at 121.9 106.71) (size 0.4) (drill 0.3) (layers "F.Cu" "B.Cu") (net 13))
 (via (at 121.95 108.113733) (size 0.4) (drill 0.3) (layers "F.Cu" "B.Cu") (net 13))
 (via (at 126.600001 98.939515) (size 0.4) (drill 0.3) (layers "F.Cu" "B.Cu") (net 13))
 (segment (start 124.386045 98.939515) (end 122 101.32556) (width 0.3) (layer "B.Cu") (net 13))
 (segment (start 121.9 106.71) (end 121.9 108.063733) (width 0.3) (layer "B.Cu") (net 13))
 (segment (start 121.999999 106.610001) (end 121.9 106.71) (width 0.3) (layer "B.Cu") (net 13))
 (segment (start 122 101.32556) (end 121.999999 106.610001) (width 0.3) (layer "B.Cu") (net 13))
 (segment (start 126.600001 98.939515) (end 124.386045 98.939515) (width 0.3) (layer "B.Cu") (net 13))
 (segment (start 121.9 108.063733) (end 121.95 108.113733) (width 0.3) (layer "B.Cu") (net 13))
 (segment (start 123 107.697412) (end 123.01179 107.685622) (width 0.3) (layer "F.Cu") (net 11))
 (segment (start 125.474929 99.316391) (end 125.474929 100.037042) (width 0.3) (layer "F.Cu") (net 11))
 (segment (start 123 112.9) (end 123 107.697412) (width 0.3) (layer "F.Cu") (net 11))
 (segment (start 125.500002 99.291318) (end 125.474929 99.316391) (width 0.3) (layer "F.Cu") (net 11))
 (segment (start 125.500002 96.189957) (end 125.500002 99.291318) (width 0.3) (layer "F.Cu") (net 11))
 (segment (start 125.5 96.189955) (end 125.500002 96.189957) (width 0.3) (layer "F.Cu") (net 11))
 (segment (start 125.474929 100.037042) (end 125.523929 100.086042) (width 0.3) (layer "F.Cu") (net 11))
 (segment (start 125.5 57.1) (end 125.5 96.189955) (width 0.3) (layer "F.Cu") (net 11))
 (via (at 123.01179 107.685622) (size 0.4) (drill 0.3) (layers "F.Cu" "B.Cu") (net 11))
 (via (at 125.523929 100.086042) (size 0.4) (drill 0.3) (layers "F.Cu" "B.Cu") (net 11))
 (segment (start 123.07 106.931471) (end 123.01179 106.873261) (width 0.3) (layer "B.Cu") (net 11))
 (segment (start 123.01179 106.873261) (end 123.01179 101.741614) (width 0.3) (layer "B.Cu") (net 11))
 (segment (start 123.01179 101.741614) (end 124.667362 100.086042) (width 0.3) (layer "B.Cu") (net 11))
 (segment (start 123.07 107.627412) (end 123.07 106.931471) (width 0.3) (layer "B.Cu") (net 11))
 (segment (start 124.667362 100.086042) (end 125.523929 100.086042) (width 0.3) (layer "B.Cu") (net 11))
 (segment (start 123.01179 107.685622) (end 123.07 107.627412) (width 0.3) (layer "B.Cu") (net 11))
 (segment (start 121 108.645636) (end 120.76 108.405636) (width 0.3) (layer "F.Cu") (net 15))
 (segment (start 127.5 57.1) (end 127.5 59.45) (width 0.3) (layer "F.Cu") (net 15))
 (segment (start 127.84 98.39) (end 127.84 98.239) (width 0.3) (layer "F.Cu") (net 15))
 (segment (start 127.68 98.079) (end 127.501 97.9) (width 0.3) (layer "F.Cu") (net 15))
 (segment (start 121 112.9) (end 121 108.645636) (width 0.3) (layer "F.Cu") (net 15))
 (segment (start 127.84 98.239) (end 127.68 98.079) (width 0.3) (layer "F.Cu") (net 15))
 (segment (start 120.76 108.405636) (end 120.76 105.88477) (width 0.3) (layer "F.Cu") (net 15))
 (segment (start 127.5 59.45) (end 127.501 59.451) (width 0.3) (layer "F.Cu") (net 15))
 (segment (start 127.501 97.9) (end 127.501 59.451) (width 0.3) (layer "F.Cu") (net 15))
 (segment (start 120.76 105.88477) (end 120.83477 105.81) (width 0.3) (layer "F.Cu") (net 15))
 (via (at 120.95 108.8) (size 0.4) (drill 0.3) (layers "F.Cu" "B.Cu") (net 15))
 (via (at 127.55 97.889516) (size 0.4) (drill 0.3) (layers "F.Cu" "B.Cu") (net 15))
 (via (at 127.84 98.39) (size 0.4) (drill 0.3) (layers "F.Cu" "B.Cu") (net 15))
 (via (at 120.83477 105.81) (size 0.4) (drill 0.3) (layers "F.Cu" "B.Cu") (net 15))
 (segment (start 127.501 97.840516) (end 127.55 97.889516) (width 0.3) (layer "B.Cu") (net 15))
 (segment (start 120.95 108.6) (end 120.95 108.8) (width 0.3) (layer "B.Cu") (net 15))
 (segment (start 120.83477 105.692336) (end 120.83477 105.81) (width 0.3) (layer "B.Cu") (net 15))
 (segment (start 120.759 105.88577) (end 120.759 107.409) (width 0.3) (layer "B.Cu") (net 15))
 (segment (start 121 100.866774) (end 121 105.527106) (width 0.3) (layer "B.Cu") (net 15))
 (segment (start 127.68 98.29) (end 127.78 98.39) (width 0.3) (layer "B.Cu") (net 15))
 (segment (start 127.441516 97.840516) (end 127.501 97.840516) (width 0.3) (layer "B.Cu") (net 15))
 (segment (start 127.55 97.889516) (end 127.610284 97.889516) (width 0.3) (layer "B.Cu") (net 15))
 (segment (start 121.586231 100.280543) (end 121 100.866774) (width 0.3) (layer "B.Cu") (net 15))
 (segment (start 127.441516 97.840516) (end 127.68 98.079) (width 0.3) (layer "B.Cu") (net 15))
 (segment (start 127.610284 97.889516) (end 127.84 98.119232) (width 0.3) (layer "B.Cu") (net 15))
 (segment (start 124.068004 97.840516) (end 121.627978 100.280542) (width 0.3) (layer "B.Cu") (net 15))
 (segment (start 120.76 107.41) (end 120.76 108.41) (width 0.3) (layer "B.Cu") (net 15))
 (segment (start 127.055221 97.840516) (end 127.25 97.840516) (width 0.3) (layer "B.Cu") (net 15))
 (segment (start 120.76 108.41) (end 120.95 108.6) (width 0.3) (layer "B.Cu") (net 15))
 (segment (start 127.25 97.840516) (end 127.25 97.86) (width 0.3) (layer "B.Cu") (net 15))
 (segment (start 126.641007 97.840516) (end 124.068004 97.840516) (width 0.3) (layer "B.Cu") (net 15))
 (segment (start 127.84 98.119232) (end 127.84 98.39) (width 0.3) (layer "B.Cu") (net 15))
 (segment (start 126.64101 97.840513) (end 126.641007 97.840516) (width 0.3) (layer "B.Cu") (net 15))
 (segment (start 120.759 107.409) (end 120.76 107.41) (width 0.3) (layer "B.Cu") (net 15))
 (segment (start 120.83477 105.81) (end 120.759 105.88577) (width 0.3) (layer "B.Cu") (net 15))
 (segment (start 127.25 97.86) (end 127.68 98.29) (width 0.3) (layer "B.Cu") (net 15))
 (segment (start 127.78 98.39) (end 127.84 98.39) (width 0.3) (layer "B.Cu") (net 15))
 (segment (start 121 105.527106) (end 120.83477 105.692336) (width 0.3) (layer "B.Cu") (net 15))
 (segment (start 121.627978 100.280542) (end 121.586231 100.280543) (width 0.3) (layer "B.Cu") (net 15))
 (segment (start 127.055221 97.840516) (end 126.64101 97.840513) (width 0.3) (layer "B.Cu") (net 15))
 (segment (start 127.25 97.840516) (end 127.441516 97.840516) (width 0.3) (layer "B.Cu") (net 15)))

